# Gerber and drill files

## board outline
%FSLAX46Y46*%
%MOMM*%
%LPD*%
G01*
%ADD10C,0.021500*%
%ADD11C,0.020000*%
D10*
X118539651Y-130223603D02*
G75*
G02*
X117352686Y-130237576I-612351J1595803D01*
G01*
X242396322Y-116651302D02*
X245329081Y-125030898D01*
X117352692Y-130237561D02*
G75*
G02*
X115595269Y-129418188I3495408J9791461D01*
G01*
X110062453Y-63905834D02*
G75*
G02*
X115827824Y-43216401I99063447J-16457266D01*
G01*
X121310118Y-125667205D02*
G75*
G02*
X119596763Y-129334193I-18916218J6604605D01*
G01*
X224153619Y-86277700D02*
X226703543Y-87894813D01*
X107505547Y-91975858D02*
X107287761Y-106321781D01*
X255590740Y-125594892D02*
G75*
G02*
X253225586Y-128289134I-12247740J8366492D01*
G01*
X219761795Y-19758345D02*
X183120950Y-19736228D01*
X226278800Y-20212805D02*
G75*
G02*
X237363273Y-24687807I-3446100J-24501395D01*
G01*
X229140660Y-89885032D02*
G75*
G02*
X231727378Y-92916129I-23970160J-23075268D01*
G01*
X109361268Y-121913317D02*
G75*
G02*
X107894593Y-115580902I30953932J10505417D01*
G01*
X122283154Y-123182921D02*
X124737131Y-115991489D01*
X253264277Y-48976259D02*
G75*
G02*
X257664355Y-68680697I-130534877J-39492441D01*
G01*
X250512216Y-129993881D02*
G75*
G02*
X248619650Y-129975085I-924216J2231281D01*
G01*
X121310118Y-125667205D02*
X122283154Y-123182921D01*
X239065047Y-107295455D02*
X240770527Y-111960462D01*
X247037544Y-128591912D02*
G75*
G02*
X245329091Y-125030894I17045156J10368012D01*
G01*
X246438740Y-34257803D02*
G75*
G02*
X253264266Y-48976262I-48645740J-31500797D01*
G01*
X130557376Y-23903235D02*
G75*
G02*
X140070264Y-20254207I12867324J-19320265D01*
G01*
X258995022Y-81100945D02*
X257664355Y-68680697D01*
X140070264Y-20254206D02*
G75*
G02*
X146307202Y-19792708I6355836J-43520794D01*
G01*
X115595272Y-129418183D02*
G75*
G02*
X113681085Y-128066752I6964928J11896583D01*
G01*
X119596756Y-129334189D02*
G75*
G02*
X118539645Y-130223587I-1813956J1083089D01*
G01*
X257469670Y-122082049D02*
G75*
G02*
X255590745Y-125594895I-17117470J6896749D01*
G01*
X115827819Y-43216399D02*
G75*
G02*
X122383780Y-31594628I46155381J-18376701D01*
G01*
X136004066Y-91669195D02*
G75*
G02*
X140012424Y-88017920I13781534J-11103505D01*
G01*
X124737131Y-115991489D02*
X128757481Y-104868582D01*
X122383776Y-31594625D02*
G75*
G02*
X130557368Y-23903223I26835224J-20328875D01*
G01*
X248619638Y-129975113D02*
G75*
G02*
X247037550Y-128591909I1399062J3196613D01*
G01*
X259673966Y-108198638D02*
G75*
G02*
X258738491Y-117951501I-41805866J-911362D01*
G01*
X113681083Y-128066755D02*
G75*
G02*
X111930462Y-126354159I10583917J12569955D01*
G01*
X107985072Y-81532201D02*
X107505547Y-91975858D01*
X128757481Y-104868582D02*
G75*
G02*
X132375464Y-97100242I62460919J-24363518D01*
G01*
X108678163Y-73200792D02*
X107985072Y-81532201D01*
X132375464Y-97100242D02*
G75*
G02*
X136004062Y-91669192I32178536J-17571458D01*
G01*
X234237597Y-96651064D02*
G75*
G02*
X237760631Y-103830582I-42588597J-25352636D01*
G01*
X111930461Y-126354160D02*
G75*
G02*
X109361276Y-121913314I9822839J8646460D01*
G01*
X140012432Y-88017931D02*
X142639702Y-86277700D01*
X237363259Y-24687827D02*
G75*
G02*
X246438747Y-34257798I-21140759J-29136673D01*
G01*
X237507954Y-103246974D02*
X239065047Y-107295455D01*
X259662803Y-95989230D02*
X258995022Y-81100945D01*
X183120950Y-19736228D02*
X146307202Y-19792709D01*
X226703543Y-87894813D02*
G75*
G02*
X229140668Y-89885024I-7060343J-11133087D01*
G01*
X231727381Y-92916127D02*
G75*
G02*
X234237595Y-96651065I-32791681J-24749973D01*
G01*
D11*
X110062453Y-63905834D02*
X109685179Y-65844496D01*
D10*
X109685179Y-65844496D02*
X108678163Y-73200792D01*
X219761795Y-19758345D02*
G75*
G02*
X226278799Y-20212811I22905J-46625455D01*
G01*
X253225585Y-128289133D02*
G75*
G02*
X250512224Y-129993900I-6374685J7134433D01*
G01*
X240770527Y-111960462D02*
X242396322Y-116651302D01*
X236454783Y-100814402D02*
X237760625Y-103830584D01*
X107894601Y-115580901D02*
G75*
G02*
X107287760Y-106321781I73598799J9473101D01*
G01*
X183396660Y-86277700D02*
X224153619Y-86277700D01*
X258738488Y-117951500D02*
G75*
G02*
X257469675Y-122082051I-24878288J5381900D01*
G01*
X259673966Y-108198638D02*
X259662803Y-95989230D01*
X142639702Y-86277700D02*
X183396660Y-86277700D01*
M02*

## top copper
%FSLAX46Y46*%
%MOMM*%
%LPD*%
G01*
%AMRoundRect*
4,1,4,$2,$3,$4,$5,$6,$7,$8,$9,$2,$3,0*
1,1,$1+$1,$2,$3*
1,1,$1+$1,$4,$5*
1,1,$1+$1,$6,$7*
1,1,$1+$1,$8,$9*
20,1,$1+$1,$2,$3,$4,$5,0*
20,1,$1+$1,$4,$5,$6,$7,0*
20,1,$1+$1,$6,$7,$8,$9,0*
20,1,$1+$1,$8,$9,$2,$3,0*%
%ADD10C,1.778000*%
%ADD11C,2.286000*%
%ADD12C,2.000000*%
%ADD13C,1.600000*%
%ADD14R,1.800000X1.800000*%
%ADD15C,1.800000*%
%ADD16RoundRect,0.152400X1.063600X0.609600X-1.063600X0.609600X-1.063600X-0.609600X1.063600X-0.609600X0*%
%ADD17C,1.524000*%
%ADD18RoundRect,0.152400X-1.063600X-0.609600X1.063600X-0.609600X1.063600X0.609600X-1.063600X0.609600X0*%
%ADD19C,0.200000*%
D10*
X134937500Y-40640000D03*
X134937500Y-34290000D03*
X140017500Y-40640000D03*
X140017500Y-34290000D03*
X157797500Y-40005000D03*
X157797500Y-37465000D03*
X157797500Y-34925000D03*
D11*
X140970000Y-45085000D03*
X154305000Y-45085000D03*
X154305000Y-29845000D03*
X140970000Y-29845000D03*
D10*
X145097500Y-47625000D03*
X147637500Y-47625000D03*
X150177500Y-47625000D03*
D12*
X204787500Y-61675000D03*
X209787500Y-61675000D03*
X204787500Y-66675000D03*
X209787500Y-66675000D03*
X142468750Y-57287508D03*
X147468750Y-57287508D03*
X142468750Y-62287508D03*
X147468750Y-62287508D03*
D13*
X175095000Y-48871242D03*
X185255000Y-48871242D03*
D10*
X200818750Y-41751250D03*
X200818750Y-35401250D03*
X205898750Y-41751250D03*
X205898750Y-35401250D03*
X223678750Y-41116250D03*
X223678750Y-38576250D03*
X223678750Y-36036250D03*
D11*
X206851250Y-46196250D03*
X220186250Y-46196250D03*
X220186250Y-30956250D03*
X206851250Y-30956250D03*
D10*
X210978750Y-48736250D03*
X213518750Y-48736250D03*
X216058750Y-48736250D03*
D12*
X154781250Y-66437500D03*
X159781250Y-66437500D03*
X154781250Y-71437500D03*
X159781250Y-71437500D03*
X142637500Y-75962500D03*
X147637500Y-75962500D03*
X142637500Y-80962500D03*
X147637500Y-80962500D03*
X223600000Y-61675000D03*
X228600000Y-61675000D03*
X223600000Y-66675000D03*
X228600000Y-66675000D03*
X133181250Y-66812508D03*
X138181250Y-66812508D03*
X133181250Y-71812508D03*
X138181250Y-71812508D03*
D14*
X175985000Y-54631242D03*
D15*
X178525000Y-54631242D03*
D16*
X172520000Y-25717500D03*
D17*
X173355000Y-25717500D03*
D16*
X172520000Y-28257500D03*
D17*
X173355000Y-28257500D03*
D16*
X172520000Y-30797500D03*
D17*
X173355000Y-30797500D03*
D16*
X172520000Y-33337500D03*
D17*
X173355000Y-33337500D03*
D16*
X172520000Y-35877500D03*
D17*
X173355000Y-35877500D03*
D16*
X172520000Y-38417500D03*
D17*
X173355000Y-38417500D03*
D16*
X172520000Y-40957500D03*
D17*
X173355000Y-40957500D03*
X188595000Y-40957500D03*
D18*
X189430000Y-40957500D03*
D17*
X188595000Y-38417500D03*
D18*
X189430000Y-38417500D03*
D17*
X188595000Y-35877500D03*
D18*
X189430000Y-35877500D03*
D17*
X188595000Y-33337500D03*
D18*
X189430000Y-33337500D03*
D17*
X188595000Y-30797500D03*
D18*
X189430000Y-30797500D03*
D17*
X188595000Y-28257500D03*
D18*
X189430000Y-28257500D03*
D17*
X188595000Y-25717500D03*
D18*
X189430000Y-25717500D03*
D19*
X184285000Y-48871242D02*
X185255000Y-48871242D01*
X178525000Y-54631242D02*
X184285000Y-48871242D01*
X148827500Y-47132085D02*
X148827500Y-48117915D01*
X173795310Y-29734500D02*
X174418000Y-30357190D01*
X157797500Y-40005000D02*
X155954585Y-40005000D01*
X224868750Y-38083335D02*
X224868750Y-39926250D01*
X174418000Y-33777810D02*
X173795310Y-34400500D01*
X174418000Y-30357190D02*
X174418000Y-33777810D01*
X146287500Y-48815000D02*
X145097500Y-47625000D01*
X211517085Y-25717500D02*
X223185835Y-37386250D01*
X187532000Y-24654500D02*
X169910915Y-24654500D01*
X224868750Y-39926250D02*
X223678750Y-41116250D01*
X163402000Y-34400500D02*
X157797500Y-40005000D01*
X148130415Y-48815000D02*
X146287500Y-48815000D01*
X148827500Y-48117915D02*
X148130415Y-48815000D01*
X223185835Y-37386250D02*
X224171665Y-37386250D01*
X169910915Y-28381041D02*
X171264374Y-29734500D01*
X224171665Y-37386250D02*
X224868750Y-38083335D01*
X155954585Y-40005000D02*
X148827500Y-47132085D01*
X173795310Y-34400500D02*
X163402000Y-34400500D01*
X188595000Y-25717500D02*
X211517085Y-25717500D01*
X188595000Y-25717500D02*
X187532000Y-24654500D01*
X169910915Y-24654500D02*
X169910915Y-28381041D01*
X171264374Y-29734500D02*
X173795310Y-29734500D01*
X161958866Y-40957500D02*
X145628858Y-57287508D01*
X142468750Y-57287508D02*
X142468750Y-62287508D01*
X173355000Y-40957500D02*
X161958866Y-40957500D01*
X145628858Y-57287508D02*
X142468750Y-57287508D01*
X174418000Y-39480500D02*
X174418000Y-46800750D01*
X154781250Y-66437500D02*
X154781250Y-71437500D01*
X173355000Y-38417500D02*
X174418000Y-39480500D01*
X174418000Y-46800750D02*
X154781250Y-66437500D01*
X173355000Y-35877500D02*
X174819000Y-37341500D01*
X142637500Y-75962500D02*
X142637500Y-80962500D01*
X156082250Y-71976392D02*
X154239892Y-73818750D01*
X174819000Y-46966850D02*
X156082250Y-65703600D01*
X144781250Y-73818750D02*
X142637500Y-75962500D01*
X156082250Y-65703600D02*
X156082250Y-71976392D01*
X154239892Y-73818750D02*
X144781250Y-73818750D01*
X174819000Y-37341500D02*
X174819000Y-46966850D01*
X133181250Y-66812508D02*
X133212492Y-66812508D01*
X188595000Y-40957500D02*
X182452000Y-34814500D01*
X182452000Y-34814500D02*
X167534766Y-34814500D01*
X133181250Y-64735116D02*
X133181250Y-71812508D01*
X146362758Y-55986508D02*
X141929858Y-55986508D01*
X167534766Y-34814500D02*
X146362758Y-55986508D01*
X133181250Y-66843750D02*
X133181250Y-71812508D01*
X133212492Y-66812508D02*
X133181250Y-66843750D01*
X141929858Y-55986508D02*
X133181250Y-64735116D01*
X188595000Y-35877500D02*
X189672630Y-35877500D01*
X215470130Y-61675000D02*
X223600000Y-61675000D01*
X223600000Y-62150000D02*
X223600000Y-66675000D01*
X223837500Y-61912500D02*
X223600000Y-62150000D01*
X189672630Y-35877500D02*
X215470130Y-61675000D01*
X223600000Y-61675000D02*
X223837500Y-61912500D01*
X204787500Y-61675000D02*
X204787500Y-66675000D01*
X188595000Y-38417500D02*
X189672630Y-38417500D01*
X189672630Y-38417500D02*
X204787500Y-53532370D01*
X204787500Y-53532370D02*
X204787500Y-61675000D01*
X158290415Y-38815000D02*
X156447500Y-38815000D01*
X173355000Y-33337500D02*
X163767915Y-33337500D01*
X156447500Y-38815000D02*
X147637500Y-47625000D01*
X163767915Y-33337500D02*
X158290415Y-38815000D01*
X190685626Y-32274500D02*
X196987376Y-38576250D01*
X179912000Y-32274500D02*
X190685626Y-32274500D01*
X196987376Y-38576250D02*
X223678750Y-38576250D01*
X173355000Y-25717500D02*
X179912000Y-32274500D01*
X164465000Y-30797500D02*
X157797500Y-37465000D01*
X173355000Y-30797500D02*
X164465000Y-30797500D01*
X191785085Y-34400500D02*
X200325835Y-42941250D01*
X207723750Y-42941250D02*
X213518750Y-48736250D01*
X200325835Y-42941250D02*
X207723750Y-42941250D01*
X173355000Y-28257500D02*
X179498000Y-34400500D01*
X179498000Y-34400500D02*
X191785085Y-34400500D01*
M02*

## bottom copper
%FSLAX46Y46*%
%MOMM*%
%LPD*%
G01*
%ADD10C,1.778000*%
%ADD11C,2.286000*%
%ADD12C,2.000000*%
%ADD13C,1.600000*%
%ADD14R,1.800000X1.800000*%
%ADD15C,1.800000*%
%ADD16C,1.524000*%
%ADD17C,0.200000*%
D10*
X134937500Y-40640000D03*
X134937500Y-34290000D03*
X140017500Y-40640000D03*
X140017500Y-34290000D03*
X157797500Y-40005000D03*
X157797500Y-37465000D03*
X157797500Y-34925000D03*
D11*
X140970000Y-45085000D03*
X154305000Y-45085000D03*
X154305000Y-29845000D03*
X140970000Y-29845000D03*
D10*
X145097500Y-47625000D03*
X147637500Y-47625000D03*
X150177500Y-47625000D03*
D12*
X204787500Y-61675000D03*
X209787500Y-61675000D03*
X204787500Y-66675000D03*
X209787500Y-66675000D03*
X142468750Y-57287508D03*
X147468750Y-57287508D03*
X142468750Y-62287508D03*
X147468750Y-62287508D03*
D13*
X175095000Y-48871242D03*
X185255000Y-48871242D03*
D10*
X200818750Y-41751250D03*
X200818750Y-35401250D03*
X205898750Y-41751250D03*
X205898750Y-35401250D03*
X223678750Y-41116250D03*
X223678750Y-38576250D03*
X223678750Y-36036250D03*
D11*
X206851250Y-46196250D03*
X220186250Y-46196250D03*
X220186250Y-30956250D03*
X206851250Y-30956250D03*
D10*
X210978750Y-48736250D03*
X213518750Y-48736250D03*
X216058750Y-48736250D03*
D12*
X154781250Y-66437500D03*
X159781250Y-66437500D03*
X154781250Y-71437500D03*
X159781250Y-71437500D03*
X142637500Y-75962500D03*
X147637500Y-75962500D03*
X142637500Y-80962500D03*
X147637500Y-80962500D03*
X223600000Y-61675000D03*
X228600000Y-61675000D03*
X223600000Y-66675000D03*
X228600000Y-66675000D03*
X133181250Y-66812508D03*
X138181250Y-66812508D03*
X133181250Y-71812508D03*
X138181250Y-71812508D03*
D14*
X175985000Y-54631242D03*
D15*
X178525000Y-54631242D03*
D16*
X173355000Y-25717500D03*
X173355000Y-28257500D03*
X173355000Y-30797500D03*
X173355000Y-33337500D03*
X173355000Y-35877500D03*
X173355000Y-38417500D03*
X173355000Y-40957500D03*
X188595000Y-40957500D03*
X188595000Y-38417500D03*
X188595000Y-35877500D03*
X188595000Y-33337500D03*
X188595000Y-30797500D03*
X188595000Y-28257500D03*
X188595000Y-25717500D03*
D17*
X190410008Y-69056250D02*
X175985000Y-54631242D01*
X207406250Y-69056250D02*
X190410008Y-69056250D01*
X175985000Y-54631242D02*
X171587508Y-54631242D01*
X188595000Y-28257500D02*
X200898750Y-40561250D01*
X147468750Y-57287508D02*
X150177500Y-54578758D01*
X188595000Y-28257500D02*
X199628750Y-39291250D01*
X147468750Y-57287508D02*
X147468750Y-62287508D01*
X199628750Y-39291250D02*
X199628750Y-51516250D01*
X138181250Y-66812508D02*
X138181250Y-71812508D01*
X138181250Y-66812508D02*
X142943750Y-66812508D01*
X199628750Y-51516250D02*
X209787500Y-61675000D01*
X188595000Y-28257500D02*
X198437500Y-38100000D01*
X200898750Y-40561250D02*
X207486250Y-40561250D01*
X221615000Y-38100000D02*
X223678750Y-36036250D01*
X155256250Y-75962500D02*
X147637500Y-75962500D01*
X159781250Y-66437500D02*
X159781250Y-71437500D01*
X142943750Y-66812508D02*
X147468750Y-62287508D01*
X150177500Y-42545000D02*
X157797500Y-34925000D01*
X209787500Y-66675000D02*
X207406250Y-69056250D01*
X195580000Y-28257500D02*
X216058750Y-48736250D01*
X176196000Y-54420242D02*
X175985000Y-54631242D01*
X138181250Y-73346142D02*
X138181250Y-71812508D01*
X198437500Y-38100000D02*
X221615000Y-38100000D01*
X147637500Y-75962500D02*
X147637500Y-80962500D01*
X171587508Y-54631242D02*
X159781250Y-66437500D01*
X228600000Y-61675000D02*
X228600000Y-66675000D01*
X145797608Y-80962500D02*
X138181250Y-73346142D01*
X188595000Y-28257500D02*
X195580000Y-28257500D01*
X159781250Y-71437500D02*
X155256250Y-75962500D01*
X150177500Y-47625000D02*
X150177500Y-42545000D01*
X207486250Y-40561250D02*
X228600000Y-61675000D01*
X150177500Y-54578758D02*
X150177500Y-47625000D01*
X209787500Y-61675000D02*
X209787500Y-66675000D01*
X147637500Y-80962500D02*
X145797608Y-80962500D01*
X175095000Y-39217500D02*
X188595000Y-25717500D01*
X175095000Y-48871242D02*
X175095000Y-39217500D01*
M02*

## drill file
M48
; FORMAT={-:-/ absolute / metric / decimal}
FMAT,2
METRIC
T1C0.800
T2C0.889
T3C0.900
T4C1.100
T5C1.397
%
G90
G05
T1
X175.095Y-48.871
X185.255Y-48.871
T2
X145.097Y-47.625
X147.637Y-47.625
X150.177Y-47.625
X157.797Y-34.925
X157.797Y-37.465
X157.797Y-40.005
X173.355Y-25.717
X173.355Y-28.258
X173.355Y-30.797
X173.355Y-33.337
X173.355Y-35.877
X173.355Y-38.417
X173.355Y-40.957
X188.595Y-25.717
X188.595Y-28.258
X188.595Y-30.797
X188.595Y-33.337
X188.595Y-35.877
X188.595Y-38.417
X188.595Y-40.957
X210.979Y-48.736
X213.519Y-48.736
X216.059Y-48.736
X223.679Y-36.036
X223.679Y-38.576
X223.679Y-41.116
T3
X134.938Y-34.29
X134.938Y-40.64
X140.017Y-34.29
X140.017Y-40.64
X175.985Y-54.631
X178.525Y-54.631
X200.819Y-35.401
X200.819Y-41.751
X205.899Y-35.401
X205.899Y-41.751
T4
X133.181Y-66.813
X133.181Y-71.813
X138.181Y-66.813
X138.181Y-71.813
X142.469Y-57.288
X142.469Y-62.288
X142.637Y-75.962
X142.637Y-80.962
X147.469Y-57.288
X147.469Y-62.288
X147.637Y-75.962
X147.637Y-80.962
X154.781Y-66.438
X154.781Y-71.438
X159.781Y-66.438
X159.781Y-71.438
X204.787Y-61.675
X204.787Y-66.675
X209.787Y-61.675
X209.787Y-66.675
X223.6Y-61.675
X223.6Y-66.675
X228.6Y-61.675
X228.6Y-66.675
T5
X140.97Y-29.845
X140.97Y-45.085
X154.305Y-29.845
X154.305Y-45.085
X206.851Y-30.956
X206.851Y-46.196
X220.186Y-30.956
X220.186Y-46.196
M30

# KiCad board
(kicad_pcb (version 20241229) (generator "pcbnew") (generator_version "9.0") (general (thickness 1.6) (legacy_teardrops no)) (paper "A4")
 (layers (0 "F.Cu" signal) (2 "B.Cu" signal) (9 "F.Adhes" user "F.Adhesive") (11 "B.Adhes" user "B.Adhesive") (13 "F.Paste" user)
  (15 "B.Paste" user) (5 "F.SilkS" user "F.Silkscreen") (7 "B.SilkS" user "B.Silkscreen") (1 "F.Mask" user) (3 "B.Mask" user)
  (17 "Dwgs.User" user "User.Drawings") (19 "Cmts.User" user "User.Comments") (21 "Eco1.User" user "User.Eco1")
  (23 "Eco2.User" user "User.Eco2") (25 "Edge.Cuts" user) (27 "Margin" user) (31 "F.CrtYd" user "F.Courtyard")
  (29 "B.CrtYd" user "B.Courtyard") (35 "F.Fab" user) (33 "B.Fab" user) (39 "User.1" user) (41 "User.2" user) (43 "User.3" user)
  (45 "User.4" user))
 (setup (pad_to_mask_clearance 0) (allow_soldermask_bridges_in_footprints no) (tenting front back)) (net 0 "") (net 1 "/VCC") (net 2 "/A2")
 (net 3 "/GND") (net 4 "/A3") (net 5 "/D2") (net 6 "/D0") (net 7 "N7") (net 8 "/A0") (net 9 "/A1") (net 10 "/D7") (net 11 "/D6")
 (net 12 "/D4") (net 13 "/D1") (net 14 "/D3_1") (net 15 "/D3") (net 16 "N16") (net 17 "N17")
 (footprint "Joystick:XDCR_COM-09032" (layer "F.Cu") (at 147.6375 37.465 90)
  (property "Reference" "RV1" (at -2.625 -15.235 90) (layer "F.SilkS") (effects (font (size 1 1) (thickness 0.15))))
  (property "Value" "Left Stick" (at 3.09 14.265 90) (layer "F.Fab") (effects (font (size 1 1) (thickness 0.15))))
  (pad "B1A" thru_hole circle (at -3.175 -12.7 90) (size 1.778 1.778) (drill 0.9) (layers "*.Cu" "*.Mask") (remove_unused_layers no)
   (solder_mask_margin 0.102))
  (pad "B1B" thru_hole circle (at 3.175 -12.7 90) (size 1.778 1.778) (drill 0.9) (layers "*.Cu" "*.Mask") (remove_unused_layers no)
   (solder_mask_margin 0.102))
  (pad "B2A" thru_hole circle (at -3.175 -7.62 90) (size 1.778 1.778) (drill 0.9) (layers "*.Cu" "*.Mask") (remove_unused_layers no)
   (solder_mask_margin 0.102))
  (pad "B2B" thru_hole circle (at 3.175 -7.62 90) (size 1.778 1.778) (drill 0.9) (layers "*.Cu" "*.Mask") (remove_unused_layers no)
   (solder_mask_margin 0.102))
  (pad "H1" thru_hole circle (at -2.54 10.16 90) (size 1.778 1.778) (drill 0.889) (layers "*.Cu" "*.Mask") (remove_unused_layers no)
   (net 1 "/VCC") (solder_mask_margin 0.102))
  (pad "H2" thru_hole circle (at 0 10.16 90) (size 1.778 1.778) (drill 0.889) (layers "*.Cu" "*.Mask") (remove_unused_layers no)
   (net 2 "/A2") (solder_mask_margin 0.102))
  (pad "H3" thru_hole circle (at 2.54 10.16 90) (size 1.778 1.778) (drill 0.889) (layers "*.Cu" "*.Mask") (remove_unused_layers no)
   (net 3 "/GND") (solder_mask_margin 0.102))
  (pad "S1" thru_hole circle (at -7.62 -6.6675 90) (size 2.286 2.286) (drill 1.397) (layers "*.Cu" "*.Mask") (remove_unused_layers no)
   (solder_mask_margin 0.102))
  (pad "S2" thru_hole circle (at -7.62 6.6675 90) (size 2.286 2.286) (drill 1.397) (layers "*.Cu" "*.Mask") (remove_unused_layers no)
   (solder_mask_margin 0.102))
  (pad "S3" thru_hole circle (at 7.62 6.6675 90) (size 2.286 2.286) (drill 1.397) (layers "*.Cu" "*.Mask") (remove_unused_layers no)
   (solder_mask_margin 0.102))
  (pad "S4" thru_hole circle (at 7.62 -6.6675 90) (size 2.286 2.286) (drill 1.397) (layers "*.Cu" "*.Mask") (remove_unused_layers no)
   (solder_mask_margin 0.102))
  (pad "V1" thru_hole circle (at -10.16 -2.54 90) (size 1.778 1.778) (drill 0.889) (layers "*.Cu" "*.Mask") (remove_unused_layers no)
   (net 1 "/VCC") (solder_mask_margin 0.102))
  (pad "V2" thru_hole circle (at -10.16 0 90) (size 1.778 1.778) (drill 0.889) (layers "*.Cu" "*.Mask") (remove_unused_layers no)
   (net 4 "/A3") (solder_mask_margin 0.102))
  (pad "V3" thru_hole circle (at -10.16 2.54 90) (size 1.778 1.778) (drill 0.889) (layers "*.Cu" "*.Mask") (remove_unused_layers no)
   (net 3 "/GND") (solder_mask_margin 0.102)))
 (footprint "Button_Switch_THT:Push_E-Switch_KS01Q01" (layer "F.Cu") (at 204.7875 61.675)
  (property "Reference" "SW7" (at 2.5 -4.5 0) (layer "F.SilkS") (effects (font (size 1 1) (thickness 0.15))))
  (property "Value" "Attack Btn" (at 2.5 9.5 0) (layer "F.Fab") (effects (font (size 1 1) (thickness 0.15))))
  (pad "1" thru_hole circle (at 0 0) (size 2 2) (drill 1.1) (layers "*.Cu" "*.Mask") (remove_unused_layers no) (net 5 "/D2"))
  (pad "2" thru_hole circle (at 5 0) (size 2 2) (drill 1.1) (layers "*.Cu" "*.Mask") (remove_unused_layers no) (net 3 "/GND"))
  (pad "3" thru_hole circle (at 0 5) (size 2 2) (drill 1.1) (layers "*.Cu" "*.Mask") (remove_unused_layers no) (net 5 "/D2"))
  (pad "4" thru_hole circle (at 5 5) (size 2 2) (drill 1.1) (layers "*.Cu" "*.Mask") (remove_unused_layers no) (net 3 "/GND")))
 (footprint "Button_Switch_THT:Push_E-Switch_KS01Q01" (layer "F.Cu") (at 142.46875 57.287508)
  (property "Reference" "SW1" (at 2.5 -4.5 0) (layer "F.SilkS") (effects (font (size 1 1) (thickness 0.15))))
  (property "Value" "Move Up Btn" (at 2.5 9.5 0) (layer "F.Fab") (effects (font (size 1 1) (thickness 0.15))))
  (pad "1" thru_hole circle (at 0 0) (size 2 2) (drill 1.1) (layers "*.Cu" "*.Mask") (remove_unused_layers no) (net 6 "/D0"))
  (pad "2" thru_hole circle (at 5 0) (size 2 2) (drill 1.1) (layers "*.Cu" "*.Mask") (remove_unused_layers no) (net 3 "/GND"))
  (pad "3" thru_hole circle (at 0 5) (size 2 2) (drill 1.1) (layers "*.Cu" "*.Mask") (remove_unused_layers no) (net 6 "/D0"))
  (pad "4" thru_hole circle (at 5 5) (size 2 2) (drill 1.1) (layers "*.Cu" "*.Mask") (remove_unused_layers no) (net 3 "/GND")))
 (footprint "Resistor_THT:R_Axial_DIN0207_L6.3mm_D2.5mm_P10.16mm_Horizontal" (layer "F.Cu") (at 175.095 48.871242)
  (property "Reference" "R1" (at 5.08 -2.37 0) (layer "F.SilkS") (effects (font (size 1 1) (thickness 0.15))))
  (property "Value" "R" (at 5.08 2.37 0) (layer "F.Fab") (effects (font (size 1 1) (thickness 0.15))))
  (pad "1" thru_hole circle (at 0 0) (size 1.6 1.6) (drill 0.8) (layers "*.Cu" "*.Mask") (remove_unused_layers no) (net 1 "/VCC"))
  (pad "2" thru_hole circle (at 10.16 0) (size 1.6 1.6) (drill 0.8) (layers "*.Cu" "*.Mask") (remove_unused_layers no) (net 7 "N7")))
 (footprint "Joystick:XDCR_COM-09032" (layer "F.Cu") (at 213.51875 38.57625 90)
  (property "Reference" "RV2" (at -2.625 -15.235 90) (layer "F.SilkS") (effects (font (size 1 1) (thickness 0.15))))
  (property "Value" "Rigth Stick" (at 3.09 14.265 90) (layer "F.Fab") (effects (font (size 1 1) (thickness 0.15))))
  (pad "B1A" thru_hole circle (at -3.175 -12.7 90) (size 1.778 1.778) (drill 0.9) (layers "*.Cu" "*.Mask") (remove_unused_layers no)
   (solder_mask_margin 0.102))
  (pad "B1B" thru_hole circle (at 3.175 -12.7 90) (size 1.778 1.778) (drill 0.9) (layers "*.Cu" "*.Mask") (remove_unused_layers no)
   (solder_mask_margin 0.102))
  (pad "B2A" thru_hole circle (at -3.175 -7.62 90) (size 1.778 1.778) (drill 0.9) (layers "*.Cu" "*.Mask") (remove_unused_layers no)
   (solder_mask_margin 0.102))
  (pad "B2B" thru_hole circle (at 3.175 -7.62 90) (size 1.778 1.778) (drill 0.9) (layers "*.Cu" "*.Mask") (remove_unused_layers no)
   (solder_mask_margin 0.102))
  (pad "H1" thru_hole circle (at -2.54 10.16 90) (size 1.778 1.778) (drill 0.889) (layers "*.Cu" "*.Mask") (remove_unused_layers no)
   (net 1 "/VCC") (solder_mask_margin 0.102))
  (pad "H2" thru_hole circle (at 0 10.16 90) (size 1.778 1.778) (drill 0.889) (layers "*.Cu" "*.Mask") (remove_unused_layers no)
   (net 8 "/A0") (solder_mask_margin 0.102))
  (pad "H3" thru_hole circle (at 2.54 10.16 90) (size 1.778 1.778) (drill 0.889) (layers "*.Cu" "*.Mask") (remove_unused_layers no)
   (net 3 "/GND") (solder_mask_margin 0.102))
  (pad "S1" thru_hole circle (at -7.62 -6.6675 90) (size 2.286 2.286) (drill 1.397) (layers "*.Cu" "*.Mask") (remove_unused_layers no)
   (solder_mask_margin 0.102))
  (pad "S2" thru_hole circle (at -7.62 6.6675 90) (size 2.286 2.286) (drill 1.397) (layers "*.Cu" "*.Mask") (remove_unused_layers no)
   (solder_mask_margin 0.102))
  (pad "S3" thru_hole circle (at 7.62 6.6675 90) (size 2.286 2.286) (drill 1.397) (layers "*.Cu" "*.Mask") (remove_unused_layers no)
   (solder_mask_margin 0.102))
  (pad "S4" thru_hole circle (at 7.62 -6.6675 90) (size 2.286 2.286) (drill 1.397) (layers "*.Cu" "*.Mask") (remove_unused_layers no)
   (solder_mask_margin 0.102))
  (pad "V1" thru_hole circle (at -10.16 -2.54 90) (size 1.778 1.778) (drill 0.889) (layers "*.Cu" "*.Mask") (remove_unused_layers no)
   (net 1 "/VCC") (solder_mask_margin 0.102))
  (pad "V2" thru_hole circle (at -10.16 0 90) (size 1.778 1.778) (drill 0.889) (layers "*.Cu" "*.Mask") (remove_unused_layers no)
   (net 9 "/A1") (solder_mask_margin 0.102))
  (pad "V3" thru_hole circle (at -10.16 2.54 90) (size 1.778 1.778) (drill 0.889) (layers "*.Cu" "*.Mask") (remove_unused_layers no)
   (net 3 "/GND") (solder_mask_margin 0.102)))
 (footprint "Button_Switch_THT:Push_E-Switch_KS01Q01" (layer "F.Cu") (at 154.78125 66.4375)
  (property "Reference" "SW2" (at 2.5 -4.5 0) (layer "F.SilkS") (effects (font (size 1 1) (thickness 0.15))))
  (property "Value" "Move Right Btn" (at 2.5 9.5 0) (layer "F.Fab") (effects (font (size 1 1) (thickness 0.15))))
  (pad "1" thru_hole circle (at 0 0) (size 2 2) (drill 1.1) (layers "*.Cu" "*.Mask") (remove_unused_layers no) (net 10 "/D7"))
  (pad "2" thru_hole circle (at 5 0) (size 2 2) (drill 1.1) (layers "*.Cu" "*.Mask") (remove_unused_layers no) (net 3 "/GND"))
  (pad "3" thru_hole circle (at 0 5) (size 2 2) (drill 1.1) (layers "*.Cu" "*.Mask") (remove_unused_layers no) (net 10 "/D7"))
  (pad "4" thru_hole circle (at 5 5) (size 2 2) (drill 1.1) (layers "*.Cu" "*.Mask") (remove_unused_layers no) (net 3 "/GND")))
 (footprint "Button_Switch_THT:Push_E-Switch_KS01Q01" (layer "F.Cu") (at 142.6375 75.9625)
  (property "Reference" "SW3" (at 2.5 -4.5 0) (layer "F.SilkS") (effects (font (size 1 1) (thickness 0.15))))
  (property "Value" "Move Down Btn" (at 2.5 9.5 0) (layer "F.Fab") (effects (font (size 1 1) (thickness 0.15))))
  (pad "1" thru_hole circle (at 0 0) (size 2 2) (drill 1.1) (layers "*.Cu" "*.Mask") (remove_unused_layers no) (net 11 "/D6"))
  (pad "2" thru_hole circle (at 5 0) (size 2 2) (drill 1.1) (layers "*.Cu" "*.Mask") (remove_unused_layers no) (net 3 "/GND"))
  (pad "3" thru_hole circle (at 0 5) (size 2 2) (drill 1.1) (layers "*.Cu" "*.Mask") (remove_unused_layers no) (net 11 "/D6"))
  (pad "4" thru_hole circle (at 5 5) (size 2 2) (drill 1.1) (layers "*.Cu" "*.Mask") (remove_unused_layers no) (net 3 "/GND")))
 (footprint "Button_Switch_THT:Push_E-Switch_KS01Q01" (layer "F.Cu") (at 223.6 61.675)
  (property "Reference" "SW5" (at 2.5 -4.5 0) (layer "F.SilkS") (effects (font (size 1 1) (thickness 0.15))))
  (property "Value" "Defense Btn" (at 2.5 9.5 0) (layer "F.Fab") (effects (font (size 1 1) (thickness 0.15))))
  (pad "1" thru_hole circle (at 0 0) (size 2 2) (drill 1.1) (layers "*.Cu" "*.Mask") (remove_unused_layers no) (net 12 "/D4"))
  (pad "2" thru_hole circle (at 5 0) (size 2 2) (drill 1.1) (layers "*.Cu" "*.Mask") (remove_unused_layers no) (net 3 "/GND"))
  (pad "3" thru_hole circle (at 0 5) (size 2 2) (drill 1.1) (layers "*.Cu" "*.Mask") (remove_unused_layers no) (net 12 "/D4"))
  (pad "4" thru_hole circle (at 5 5) (size 2 2) (drill 1.1) (layers "*.Cu" "*.Mask") (remove_unused_layers no) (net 3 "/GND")))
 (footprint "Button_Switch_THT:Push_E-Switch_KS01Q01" (layer "F.Cu") (at 133.18125 66.812508)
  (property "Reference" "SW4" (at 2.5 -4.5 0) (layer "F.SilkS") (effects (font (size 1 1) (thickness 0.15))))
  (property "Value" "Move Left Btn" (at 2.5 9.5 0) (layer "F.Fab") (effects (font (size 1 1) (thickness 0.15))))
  (pad "1" thru_hole circle (at 0 0) (size 2 2) (drill 1.1) (layers "*.Cu" "*.Mask") (remove_unused_layers no) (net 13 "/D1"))
  (pad "2" thru_hole circle (at 5 0) (size 2 2) (drill 1.1) (layers "*.Cu" "*.Mask") (remove_unused_layers no) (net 3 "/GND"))
  (pad "3" thru_hole circle (at 0 5) (size 2 2) (drill 1.1) (layers "*.Cu" "*.Mask") (remove_unused_layers no) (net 13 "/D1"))
  (pad "4" thru_hole circle (at 5 5) (size 2 2) (drill 1.1) (layers "*.Cu" "*.Mask") (remove_unused_layers no) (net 3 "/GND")))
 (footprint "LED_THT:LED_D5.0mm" (layer "F.Cu") (at 175.985 54.631242)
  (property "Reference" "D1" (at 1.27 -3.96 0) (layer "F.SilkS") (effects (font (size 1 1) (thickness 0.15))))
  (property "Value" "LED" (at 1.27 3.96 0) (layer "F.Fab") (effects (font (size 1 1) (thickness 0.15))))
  (pad "1" thru_hole rect (at 0 0) (size 1.8 1.8) (drill 0.9) (layers "*.Cu" "*.Mask") (remove_unused_layers no) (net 3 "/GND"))
  (pad "2" thru_hole circle (at 2.54 0) (size 1.8 1.8) (drill 0.9) (layers "*.Cu" "*.Mask") (remove_unused_layers no) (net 7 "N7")))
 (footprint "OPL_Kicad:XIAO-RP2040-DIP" (layer "F.Cu") (at 180.975 33.3375)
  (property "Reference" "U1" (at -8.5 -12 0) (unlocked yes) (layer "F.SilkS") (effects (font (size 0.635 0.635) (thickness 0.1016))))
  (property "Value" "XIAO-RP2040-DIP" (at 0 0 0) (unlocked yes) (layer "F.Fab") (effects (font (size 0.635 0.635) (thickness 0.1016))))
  (pad "1" smd roundrect (at -8.455 -7.62 180) (size 2.432 1.524) (layers "F.Cu" "F.Mask") (roundrect_rratio 0.1) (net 8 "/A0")
   (thermal_bridge_angle 45))
  (pad "1" thru_hole circle (at -7.62 -7.62 180) (size 1.524 1.524) (drill 0.889) (layers "*.Cu" "*.Mask") (remove_unused_layers no)
   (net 8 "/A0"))
  (pad "2" smd roundrect (at -8.455 -5.08 180) (size 2.432 1.524) (layers "F.Cu" "F.Mask") (roundrect_rratio 0.1) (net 9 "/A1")
   (thermal_bridge_angle 45))
  (pad "2" thru_hole circle (at -7.62 -5.08 180) (size 1.524 1.524) (drill 0.889) (layers "*.Cu" "*.Mask") (remove_unused_layers no)
   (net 9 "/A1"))
  (pad "3" smd roundrect (at -8.455 -2.54 180) (size 2.432 1.524) (layers "F.Cu" "F.Mask") (roundrect_rratio 0.1) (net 2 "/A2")
   (thermal_bridge_angle 45))
  (pad "3" thru_hole circle (at -7.62 -2.54 180) (size 1.524 1.524) (drill 0.889) (layers "*.Cu" "*.Mask") (remove_unused_layers no)
   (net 2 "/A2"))
  (pad "4" smd roundrect (at -8.455 0 180) (size 2.432 1.524) (layers "F.Cu" "F.Mask") (roundrect_rratio 0.1) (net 4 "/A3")
   (thermal_bridge_angle 45))
  (pad "4" thru_hole circle (at -7.62 0 180) (size 1.524 1.524) (drill 0.889) (layers "*.Cu" "*.Mask") (remove_unused_layers no)
   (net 4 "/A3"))
  (pad "5" smd roundrect (at -8.455 2.54 180) (size 2.432 1.524) (layers "F.Cu" "F.Mask") (roundrect_rratio 0.1) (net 11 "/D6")
   (thermal_bridge_angle 45))
  (pad "5" thru_hole circle (at -7.62 2.54 180) (size 1.524 1.524) (drill 0.889) (layers "*.Cu" "*.Mask") (remove_unused_layers no)
   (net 11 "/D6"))
  (pad "6" smd roundrect (at -8.455 5.08 180) (size 2.432 1.524) (layers "F.Cu" "F.Mask") (roundrect_rratio 0.1) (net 10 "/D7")
   (thermal_bridge_angle 45))
  (pad "6" thru_hole circle (at -7.62 5.08 180) (size 1.524 1.524) (drill 0.889) (layers "*.Cu" "*.Mask") (remove_unused_layers no)
   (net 10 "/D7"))
  (pad "7" smd roundrect (at -8.455 7.62 180) (size 2.432 1.524) (layers "F.Cu" "F.Mask") (roundrect_rratio 0.1) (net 6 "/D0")
   (thermal_bridge_angle 45))
  (pad "7" thru_hole circle (at -7.62 7.62 180) (size 1.524 1.524) (drill 0.889) (layers "*.Cu" "*.Mask") (remove_unused_layers no)
   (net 6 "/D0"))
  (pad "8" thru_hole circle (at 7.62 7.62) (size 1.524 1.524) (drill 0.889) (layers "*.Cu" "*.Mask") (remove_unused_layers no)
   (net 13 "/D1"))
  (pad "8" smd roundrect (at 8.455 7.62) (size 2.432 1.524) (layers "F.Cu" "F.Mask") (roundrect_rratio 0.1) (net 13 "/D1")
   (thermal_bridge_angle 45))
  (pad "9" thru_hole circle (at 7.62 5.08) (size 1.524 1.524) (drill 0.889) (layers "*.Cu" "*.Mask") (remove_unused_layers no) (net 5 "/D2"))
  (pad "9" smd roundrect (at 8.455 5.08) (size 2.432 1.524) (layers "F.Cu" "F.Mask") (roundrect_rratio 0.1) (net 5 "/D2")
   (thermal_bridge_angle 45))
  (pad "10" thru_hole circle (at 7.62 2.54) (size 1.524 1.524) (drill 0.889) (layers "*.Cu" "*.Mask") (remove_unused_layers no)
   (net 12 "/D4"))
  (pad "10" smd roundrect (at 8.455 2.54) (size 2.432 1.524) (layers "F.Cu" "F.Mask") (roundrect_rratio 0.1) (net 12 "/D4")
   (thermal_bridge_angle 45))
  (pad "11" thru_hole circle (at 7.62 0) (size 1.524 1.524) (drill 0.889) (layers "*.Cu" "*.Mask") (remove_unused_layers no)
   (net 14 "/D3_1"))
  (pad "11" smd roundrect (at 8.455 0) (size 2.432 1.524) (layers "F.Cu" "F.Mask") (roundrect_rratio 0.1) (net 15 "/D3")
   (thermal_bridge_angle 45))
  (pad "12" thru_hole circle (at 7.62 -2.54) (size 1.524 1.524) (drill 0.889) (layers "*.Cu" "*.Mask") (remove_unused_layers no)
   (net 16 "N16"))
  (pad "12" smd roundrect (at 8.455 -2.54) (size 2.432 1.524) (layers "F.Cu" "F.Mask") (roundrect_rratio 0.1) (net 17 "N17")
   (thermal_bridge_angle 45))
  (pad "13" thru_hole circle (at 7.62 -5.08) (size 1.524 1.524) (drill 0.889) (layers "*.Cu" "*.Mask") (remove_unused_layers no)
   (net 3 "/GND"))
  (pad "13" smd roundrect (at 8.455 -5.08) (size 2.432 1.524) (layers "F.Cu" "F.Mask") (roundrect_rratio 0.1) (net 3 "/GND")
   (thermal_bridge_angle 45))
  (pad "14" thru_hole circle (at 7.62 -7.62) (size 1.524 1.524) (drill 0.889) (layers "*.Cu" "*.Mask") (remove_unused_layers no)
   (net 1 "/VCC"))
  (pad "14" smd roundrect (at 8.455 -7.62) (size 2.432 1.524) (layers "F.Cu" "F.Mask") (roundrect_rratio 0.1) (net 1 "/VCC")
   (thermal_bridge_angle 45)))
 (gr_arc (start 118.539651 130.223603) (mid 117.947424 130.336928) (end 117.352692 130.237561) (stroke (width 0.0215) (type default))
  (layer "Edge.Cuts"))
 (gr_line (start 242.396322 116.651302) (end 245.329081 125.030898) (stroke (width 0.0215) (type default)) (layer "Edge.Cuts"))
 (gr_arc (start 117.352692 130.237561) (mid 116.454838 129.868933) (end 115.595272 129.418183) (stroke (width 0.0215) (type default))
  (layer "Edge.Cuts"))
 (gr_arc (start 110.062453 63.905834) (mid 112.390423 53.406539) (end 115.827819 43.216399) (stroke (width 0.0215) (type default))
  (layer "Edge.Cuts"))
 (gr_arc (start 121.310118 125.667205) (mid 120.546271 127.544073) (end 119.596756 129.334189) (stroke (width 0.0215) (type default))
  (layer "Edge.Cuts"))
 (gr_line (start 224.153619 86.2777) (end 226.703543 87.894813) (stroke (width 0.0215) (type default)) (layer "Edge.Cuts"))
 (gr_line (start 107.505547 91.975858) (end 107.287761 106.321781) (stroke (width 0.0215) (type default)) (layer "Edge.Cuts"))
 (gr_arc (start 255.59074 125.594892) (mid 254.489863 127.013734) (end 253.225585 128.289133) (stroke (width 0.0215) (type default))
  (layer "Edge.Cuts"))
 (gr_line (start 219.761795 19.758345) (end 183.12095 19.736228) (stroke (width 0.0215) (type default)) (layer "Edge.Cuts"))
 (gr_arc (start 226.2788 20.212805) (mid 232.09534 21.770859) (end 237.363259 24.687827) (stroke (width 0.0215) (type default))
  (layer "Edge.Cuts"))
 (gr_arc (start 229.14066 89.885032) (mid 230.479438 91.36182) (end 231.727381 92.916127) (stroke (width 0.0215) (type default))
  (layer "Edge.Cuts"))
 (gr_arc (start 109.361268 121.913317) (mid 108.470143 118.783656) (end 107.894601 115.580901) (stroke (width 0.0215) (type default))
  (layer "Edge.Cuts"))
 (gr_line (start 122.283154 123.182921) (end 124.737131 115.991489) (stroke (width 0.0215) (type default)) (layer "Edge.Cuts"))
 (gr_arc (start 253.264277 48.976259) (mid 255.829453 58.746941) (end 257.664355 68.680697) (stroke (width 0.0215) (type default))
  (layer "Edge.Cuts"))
 (gr_arc (start 250.512216 129.993881) (mid 249.564011 130.17761) (end 248.619638 129.975113) (stroke (width 0.0215) (type default))
  (layer "Edge.Cuts"))
 (gr_line (start 121.310118 125.667205) (end 122.283154 123.182921) (stroke (width 0.0215) (type default)) (layer "Edge.Cuts"))
 (gr_line (start 239.065047 107.295455) (end 240.770527 111.960462) (stroke (width 0.0215) (type default)) (layer "Edge.Cuts"))
 (gr_arc (start 247.037544 128.591912) (mid 246.094974 126.853787) (end 245.329081 125.030898) (stroke (width 0.0215) (type default))
  (layer "Edge.Cuts"))
 (gr_arc (start 246.43874 34.257803) (mid 250.369103 41.377002) (end 253.264277 48.976259) (stroke (width 0.0215) (type default))
  (layer "Edge.Cuts"))
 (gr_arc (start 130.557376 23.903235) (mid 135.111143 21.55035) (end 140.070264 20.254206) (stroke (width 0.0215) (type default))
  (layer "Edge.Cuts"))
 (gr_line (start 258.995022 81.100945) (end 257.664355 68.680697) (stroke (width 0.0215) (type default)) (layer "Edge.Cuts"))
 (gr_arc (start 140.070264 20.254206) (mid 143.18052 19.912461) (end 146.307202 19.792709) (stroke (width 0.0215) (type default))
  (layer "Edge.Cuts"))
 (gr_arc (start 115.595272 129.418183) (mid 114.609412 128.783213) (end 113.681083 128.066755) (stroke (width 0.0215) (type default))
  (layer "Edge.Cuts"))
 (gr_arc (start 119.596756 129.334189) (mid 119.142954 129.867742) (end 118.539651 130.223603) (stroke (width 0.0215) (type default))
  (layer "Edge.Cuts"))
 (gr_arc (start 257.46967 122.082049) (mid 256.625272 123.889319) (end 255.59074 125.594892) (stroke (width 0.0215) (type default))
  (layer "Edge.Cuts"))
 (gr_arc (start 115.827819 43.216399) (mid 118.713834 37.184402) (end 122.383776 31.594625) (stroke (width 0.0215) (type default))
  (layer "Edge.Cuts"))
 (gr_arc (start 136.004066 91.669195) (mid 137.867591 89.689148) (end 140.012432 88.017931) (stroke (width 0.0215) (type default))
  (layer "Edge.Cuts"))
 (gr_line (start 124.737131 115.991489) (end 128.757481 104.868582) (stroke (width 0.0215) (type default)) (layer "Edge.Cuts"))
 (gr_arc (start 122.383776 31.594625) (mid 126.147802 27.405919) (end 130.557376 23.903235) (stroke (width 0.0215) (type default))
  (layer "Edge.Cuts"))
 (gr_arc (start 248.619638 129.975113) (mid 247.721986 129.405448) (end 247.037544 128.591912) (stroke (width 0.0215) (type default))
  (layer "Edge.Cuts"))
 (gr_arc (start 259.673966 108.198638) (mid 259.492856 113.102562) (end 258.738488 117.9515) (stroke (width 0.0215) (type default))
  (layer "Edge.Cuts"))
 (gr_arc (start 113.681083 128.066755) (mid 112.773823 127.243116) (end 111.930461 126.35416) (stroke (width 0.0215) (type default))
  (layer "Edge.Cuts"))
 (gr_line (start 107.985072 81.532201) (end 107.505547 91.975858) (stroke (width 0.0215) (type default)) (layer "Edge.Cuts"))
 (gr_arc (start 128.757481 104.868582) (mid 130.442228 100.926547) (end 132.375464 97.100242) (stroke (width 0.0215) (type default))
  (layer "Edge.Cuts"))
 (gr_line (start 108.678163 73.200792) (end 107.985072 81.532201) (stroke (width 0.0215) (type default)) (layer "Edge.Cuts"))
 (gr_arc (start 132.375464 97.100242) (mid 134.06858 94.303752) (end 136.004066 91.669195) (stroke (width 0.0215) (type default))
  (layer "Edge.Cuts"))
 (gr_arc (start 234.237597 96.651064) (mid 236.144154 100.169651) (end 237.760625 103.830584) (stroke (width 0.0215) (type default))
  (layer "Edge.Cuts"))
 (gr_arc (start 111.930461 126.35416) (mid 110.426103 124.260878) (end 109.361268 121.913317) (stroke (width 0.0215) (type default))
  (layer "Edge.Cuts"))
 (gr_line (start 140.012432 88.017931) (end 142.639702 86.2777) (stroke (width 0.0215) (type default)) (layer "Edge.Cuts"))
 (gr_arc (start 237.363259 24.687827) (mid 242.343017 29.053637) (end 246.43874 34.257803) (stroke (width 0.0215) (type default))
  (layer "Edge.Cuts"))
 (gr_line (start 237.507954 103.246974) (end 239.065047 107.295455) (stroke (width 0.0215) (type default)) (layer "Edge.Cuts"))
 (gr_line (start 259.662803 95.98923) (end 258.995022 81.100945) (stroke (width 0.0215) (type default)) (layer "Edge.Cuts"))
 (gr_line (start 183.12095 19.736228) (end 146.307202 19.792709) (stroke (width 0.0215) (type default)) (layer "Edge.Cuts"))
 (gr_arc (start 226.703543 87.894813) (mid 227.981692 88.816951) (end 229.14066 89.885032) (stroke (width 0.0215) (type default))
  (layer "Edge.Cuts"))
 (gr_arc (start 231.727381 92.916127) (mid 233.033666 94.7492) (end 234.237597 96.651064) (stroke (width 0.0215) (type default))
  (layer "Edge.Cuts"))
 (gr_line (start 110.062453 63.905834) (end 109.685179 65.844496) (stroke (width 0.02) (type solid)) (layer "Edge.Cuts"))
 (gr_line (start 109.685179 65.844496) (end 108.678163 73.200792) (stroke (width 0.0215) (type default)) (layer "Edge.Cuts"))
 (gr_arc (start 219.761795 19.758345) (mid 223.028267 19.871295) (end 226.2788 20.212805) (stroke (width 0.0215) (type default))
  (layer "Edge.Cuts"))
 (gr_arc (start 253.225585 128.289133) (mid 251.94078 129.255914) (end 250.512216 129.993881) (stroke (width 0.0215) (type default))
  (layer "Edge.Cuts"))
 (gr_line (start 240.770527 111.960462) (end 242.396322 116.651302) (stroke (width 0.0215) (type default)) (layer "Edge.Cuts"))
 (gr_line (start 236.454783 100.814402) (end 237.760625 103.830584) (stroke (width 0.0215) (type default)) (layer "Edge.Cuts"))
 (gr_arc (start 107.894601 115.580901) (mid 107.446315 110.960835) (end 107.287761 106.321781) (stroke (width 0.0215) (type default))
  (layer "Edge.Cuts"))
 (gr_line (start 183.39666 86.2777) (end 224.153619 86.2777) (stroke (width 0.0215) (type default)) (layer "Edge.Cuts"))
 (gr_arc (start 258.738488 117.9515) (mid 258.191888 120.043747) (end 257.46967 122.082049) (stroke (width 0.0215) (type default))
  (layer "Edge.Cuts"))
 (gr_line (start 259.673966 108.198638) (end 259.662803 95.98923) (stroke (width 0.0215) (type default)) (layer "Edge.Cuts"))
 (gr_line (start 142.639702 86.2777) (end 183.39666 86.2777) (stroke (width 0.0215) (type default)) (layer "Edge.Cuts"))
 (segment (start 184.285 48.871242) (end 185.255 48.871242) (width 0.2) (layer "F.Cu") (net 7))
 (segment (start 178.525 54.631242) (end 184.285 48.871242) (width 0.2) (layer "F.Cu") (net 7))
 (segment (start 190.410008 69.05625) (end 175.985 54.631242) (width 0.2) (layer "B.Cu") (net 3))
 (segment (start 207.40625 69.05625) (end 190.410008 69.05625) (width 0.2) (layer "B.Cu") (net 3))
 (segment (start 175.985 54.631242) (end 171.587508 54.631242) (width 0.2) (layer "B.Cu") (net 3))
 (segment (start 188.595 28.2575) (end 200.89875 40.56125) (width 0.2) (layer "B.Cu") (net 3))
 (segment (start 147.46875 57.287508) (end 150.1775 54.578758) (width 0.2) (layer "B.Cu") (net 3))
 (segment (start 188.595 28.2575) (end 199.62875 39.29125) (width 0.2) (layer "B.Cu") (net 3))
 (segment (start 147.46875 57.287508) (end 147.46875 62.287508) (width 0.2) (layer "B.Cu") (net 3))
 (segment (start 199.62875 39.29125) (end 199.62875 51.51625) (width 0.2) (layer "B.Cu") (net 3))
 (segment (start 138.18125 66.812508) (end 138.18125 71.812508) (width 0.2) (layer "B.Cu") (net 3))
 (segment (start 138.18125 66.812508) (end 142.94375 66.812508) (width 0.2) (layer "B.Cu") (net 3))
 (segment (start 199.62875 51.51625) (end 209.7875 61.675) (width 0.2) (layer "B.Cu") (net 3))
 (segment (start 188.595 28.2575) (end 198.4375 38.1) (width 0.2) (layer "B.Cu") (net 3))
 (segment (start 200.89875 40.56125) (end 207.48625 40.56125) (width 0.2) (layer "B.Cu") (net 3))
 (segment (start 221.615 38.1) (end 223.67875 36.03625) (width 0.2) (layer "B.Cu") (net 3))
 (segment (start 155.25625 75.9625) (end 147.6375 75.9625) (width 0.2) (layer "B.Cu") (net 3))
 (segment (start 159.78125 66.4375) (end 159.78125 71.4375) (width 0.2) (layer "B.Cu") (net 3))
 (segment (start 142.94375 66.812508) (end 147.46875 62.287508) (width 0.2) (layer "B.Cu") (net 3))
 (segment (start 150.1775 42.545) (end 157.7975 34.925) (width 0.2) (layer "B.Cu") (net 3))
 (segment (start 209.7875 66.675) (end 207.40625 69.05625) (width 0.2) (layer "B.Cu") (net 3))
 (segment (start 195.58 28.2575) (end 216.05875 48.73625) (width 0.2) (layer "B.Cu") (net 3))
 (segment (start 176.196 54.420242) (end 175.985 54.631242) (width 0.2) (layer "B.Cu") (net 3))
 (segment (start 138.18125 73.346142) (end 138.18125 71.812508) (width 0.2) (layer "B.Cu") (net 3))
 (segment (start 198.4375 38.1) (end 221.615 38.1) (width 0.2) (layer "B.Cu") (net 3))
 (segment (start 147.6375 75.9625) (end 147.6375 80.9625) (width 0.2) (layer "B.Cu") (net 3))
 (segment (start 171.587508 54.631242) (end 159.78125 66.4375) (width 0.2) (layer "B.Cu") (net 3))
 (segment (start 228.6 61.675) (end 228.6 66.675) (width 0.2) (layer "B.Cu") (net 3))
 (segment (start 145.797608 80.9625) (end 138.18125 73.346142) (width 0.2) (layer "B.Cu") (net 3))
 (segment (start 188.595 28.2575) (end 195.58 28.2575) (width 0.2) (layer "B.Cu") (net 3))
 (segment (start 159.78125 71.4375) (end 155.25625 75.9625) (width 0.2) (layer "B.Cu") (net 3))
 (segment (start 150.1775 47.625) (end 150.1775 42.545) (width 0.2) (layer "B.Cu") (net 3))
 (segment (start 207.48625 40.56125) (end 228.6 61.675) (width 0.2) (layer "B.Cu") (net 3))
 (segment (start 150.1775 54.578758) (end 150.1775 47.625) (width 0.2) (layer "B.Cu") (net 3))
 (segment (start 209.7875 61.675) (end 209.7875 66.675) (width 0.2) (layer "B.Cu") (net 3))
 (segment (start 147.6375 80.9625) (end 145.797608 80.9625) (width 0.2) (layer "B.Cu") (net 3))
 (segment (start 148.8275 47.132085) (end 148.8275 48.117915) (width 0.2) (layer "F.Cu") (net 1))
 (segment (start 173.79531 29.7345) (end 174.418 30.35719) (width 0.2) (layer "F.Cu") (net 1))
 (segment (start 157.7975 40.005) (end 155.954585 40.005) (width 0.2) (layer "F.Cu") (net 1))
 (segment (start 224.86875 38.083335) (end 224.86875 39.92625) (width 0.2) (layer "F.Cu") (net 1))
 (segment (start 174.418 33.77781) (end 173.79531 34.4005) (width 0.2) (layer "F.Cu") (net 1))
 (segment (start 174.418 30.35719) (end 174.418 33.77781) (width 0.2) (layer "F.Cu") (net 1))
 (segment (start 146.2875 48.815) (end 145.0975 47.625) (width 0.2) (layer "F.Cu") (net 1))
 (segment (start 211.517085 25.7175) (end 223.185835 37.38625) (width 0.2) (layer "F.Cu") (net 1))
 (segment (start 187.532 24.6545) (end 169.910915 24.6545) (width 0.2) (layer "F.Cu") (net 1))
 (segment (start 224.86875 39.92625) (end 223.67875 41.11625) (width 0.2) (layer "F.Cu") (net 1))
 (segment (start 163.402 34.4005) (end 157.7975 40.005) (width 0.2) (layer "F.Cu") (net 1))
 (segment (start 148.130415 48.815) (end 146.2875 48.815) (width 0.2) (layer "F.Cu") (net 1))
 (segment (start 148.8275 48.117915) (end 148.130415 48.815) (width 0.2) (layer "F.Cu") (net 1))
 (segment (start 223.185835 37.38625) (end 224.171665 37.38625) (width 0.2) (layer "F.Cu") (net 1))
 (segment (start 169.910915 28.381041) (end 171.264374 29.7345) (width 0.2) (layer "F.Cu") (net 1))
 (segment (start 224.171665 37.38625) (end 224.86875 38.083335) (width 0.2) (layer "F.Cu") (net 1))
 (segment (start 155.954585 40.005) (end 148.8275 47.132085) (width 0.2) (layer "F.Cu") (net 1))
 (segment (start 173.79531 34.4005) (end 163.402 34.4005) (width 0.2) (layer "F.Cu") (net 1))
 (segment (start 188.595 25.7175) (end 211.517085 25.7175) (width 0.2) (layer "F.Cu") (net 1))
 (segment (start 188.595 25.7175) (end 187.532 24.6545) (width 0.2) (layer "F.Cu") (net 1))
 (segment (start 169.910915 24.6545) (end 169.910915 28.381041) (width 0.2) (layer "F.Cu") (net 1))
 (segment (start 171.264374 29.7345) (end 173.79531 29.7345) (width 0.2) (layer "F.Cu") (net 1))
 (segment (start 175.095 39.2175) (end 188.595 25.7175) (width 0.2) (layer "B.Cu") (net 1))
 (segment (start 175.095 48.871242) (end 175.095 39.2175) (width 0.2) (layer "B.Cu") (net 1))
 (segment (start 161.958866 40.9575) (end 145.628858 57.287508) (width 0.2) (layer "F.Cu") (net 6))
 (segment (start 142.46875 57.287508) (end 142.46875 62.287508) (width 0.2) (layer "F.Cu") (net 6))
 (segment (start 173.355 40.9575) (end 161.958866 40.9575) (width 0.2) (layer "F.Cu") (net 6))
 (segment (start 145.628858 57.287508) (end 142.46875 57.287508) (width 0.2) (layer "F.Cu") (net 6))
 (segment (start 174.418 39.4805) (end 174.418 46.80075) (width 0.2) (layer "F.Cu") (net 10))
 (segment (start 154.78125 66.4375) (end 154.78125 71.4375) (width 0.2) (layer "F.Cu") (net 10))
 (segment (start 173.355 38.4175) (end 174.418 39.4805) (width 0.2) (layer "F.Cu") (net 10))
 (segment (start 174.418 46.80075) (end 154.78125 66.4375) (width 0.2) (layer "F.Cu") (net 10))
 (segment (start 173.355 35.8775) (end 174.819 37.3415) (width 0.2) (layer "F.Cu") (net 11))
 (segment (start 142.6375 75.9625) (end 142.6375 80.9625) (width 0.2) (layer "F.Cu") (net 11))
 (segment (start 156.08225 71.976392) (end 154.239892 73.81875) (width 0.2) (layer "F.Cu") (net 11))
 (segment (start 174.819 46.96685) (end 156.08225 65.7036) (width 0.2) (layer "F.Cu") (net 11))
 (segment (start 144.78125 73.81875) (end 142.6375 75.9625) (width 0.2) (layer "F.Cu") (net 11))
 (segment (start 156.08225 65.7036) (end 156.08225 71.976392) (width 0.2) (layer "F.Cu") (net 11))
 (segment (start 154.239892 73.81875) (end 144.78125 73.81875) (width 0.2) (layer "F.Cu") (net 11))
 (segment (start 174.819 37.3415) (end 174.819 46.96685) (width 0.2) (layer "F.Cu") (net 11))
 (segment (start 133.18125 66.812508) (end 133.212492 66.812508) (width 0.2) (layer "F.Cu") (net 13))
 (segment (start 188.595 40.9575) (end 182.452 34.8145) (width 0.2) (layer "F.Cu") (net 13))
 (segment (start 182.452 34.8145) (end 167.534766 34.8145) (width 0.2) (layer "F.Cu") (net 13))
 (segment (start 133.18125 64.735116) (end 133.18125 71.812508) (width 0.2) (layer "F.Cu") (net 13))
 (segment (start 146.362758 55.986508) (end 141.929858 55.986508) (width 0.2) (layer "F.Cu") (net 13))
 (segment (start 167.534766 34.8145) (end 146.362758 55.986508) (width 0.2) (layer "F.Cu") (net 13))
 (segment (start 133.18125 66.84375) (end 133.18125 71.812508) (width 0.2) (layer "F.Cu") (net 13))
 (segment (start 133.212492 66.812508) (end 133.18125 66.84375) (width 0.2) (layer "F.Cu") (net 13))
 (segment (start 141.929858 55.986508) (end 133.18125 64.735116) (width 0.2) (layer "F.Cu") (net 13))
 (segment (start 188.595 35.8775) (end 189.67263 35.8775) (width 0.2) (layer "F.Cu") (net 12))
 (segment (start 215.47013 61.675) (end 223.6 61.675) (width 0.2) (layer "F.Cu") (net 12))
 (segment (start 223.6 62.15) (end 223.6 66.675) (width 0.2) (layer "F.Cu") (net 12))
 (segment (start 223.8375 61.9125) (end 223.6 62.15) (width 0.2) (layer "F.Cu") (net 12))
 (segment (start 189.67263 35.8775) (end 215.47013 61.675) (width 0.2) (layer "F.Cu") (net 12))
 (segment (start 223.6 61.675) (end 223.8375 61.9125) (width 0.2) (layer "F.Cu") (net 12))
 (segment (start 204.7875 61.675) (end 204.7875 66.675) (width 0.2) (layer "F.Cu") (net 5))
 (segment (start 188.595 38.4175) (end 189.67263 38.4175) (width 0.2) (layer "F.Cu") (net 5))
 (segment (start 189.67263 38.4175) (end 204.7875 53.53237) (width 0.2) (layer "F.Cu") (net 5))
 (segment (start 204.7875 53.53237) (end 204.7875 61.675) (width 0.2) (layer "F.Cu") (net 5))
 (segment (start 158.290415 38.815) (end 156.4475 38.815) (width 0.2) (layer "F.Cu") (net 4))
 (segment (start 173.355 33.3375) (end 163.767915 33.3375) (width 0.2) (layer "F.Cu") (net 4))
 (segment (start 156.4475 38.815) (end 147.6375 47.625) (width 0.2) (layer "F.Cu") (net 4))
 (segment (start 163.767915 33.3375) (end 158.290415 38.815) (width 0.2) (layer "F.Cu") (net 4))
 (segment (start 190.685626 32.2745) (end 196.987376 38.57625) (width 0.2) (layer "F.Cu") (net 8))
 (segment (start 179.912 32.2745) (end 190.685626 32.2745) (width 0.2) (layer "F.Cu") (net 8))
 (segment (start 196.987376 38.57625) (end 223.67875 38.57625) (width 0.2) (layer "F.Cu") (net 8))
 (segment (start 173.355 25.7175) (end 179.912 32.2745) (width 0.2) (layer "F.Cu") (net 8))
 (segment (start 164.465 30.7975) (end 157.7975 37.465) (width 0.2) (layer "F.Cu") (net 2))
 (segment (start 173.355 30.7975) (end 164.465 30.7975) (width 0.2) (layer "F.Cu") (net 2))
 (segment (start 191.785085 34.4005) (end 200.325835 42.94125) (width 0.2) (layer "F.Cu") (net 9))
 (segment (start 207.72375 42.94125) (end 213.51875 48.73625) (width 0.2) (layer "F.Cu") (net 9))
 (segment (start 200.325835 42.94125) (end 207.72375 42.94125) (width 0.2) (layer "F.Cu") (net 9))
 (segment (start 173.355 28.2575) (end 179.498 34.4005) (width 0.2) (layer "F.Cu") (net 9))
 (segment (start 179.498 34.4005) (end 191.785085 34.4005) (width 0.2) (layer "F.Cu") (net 9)))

